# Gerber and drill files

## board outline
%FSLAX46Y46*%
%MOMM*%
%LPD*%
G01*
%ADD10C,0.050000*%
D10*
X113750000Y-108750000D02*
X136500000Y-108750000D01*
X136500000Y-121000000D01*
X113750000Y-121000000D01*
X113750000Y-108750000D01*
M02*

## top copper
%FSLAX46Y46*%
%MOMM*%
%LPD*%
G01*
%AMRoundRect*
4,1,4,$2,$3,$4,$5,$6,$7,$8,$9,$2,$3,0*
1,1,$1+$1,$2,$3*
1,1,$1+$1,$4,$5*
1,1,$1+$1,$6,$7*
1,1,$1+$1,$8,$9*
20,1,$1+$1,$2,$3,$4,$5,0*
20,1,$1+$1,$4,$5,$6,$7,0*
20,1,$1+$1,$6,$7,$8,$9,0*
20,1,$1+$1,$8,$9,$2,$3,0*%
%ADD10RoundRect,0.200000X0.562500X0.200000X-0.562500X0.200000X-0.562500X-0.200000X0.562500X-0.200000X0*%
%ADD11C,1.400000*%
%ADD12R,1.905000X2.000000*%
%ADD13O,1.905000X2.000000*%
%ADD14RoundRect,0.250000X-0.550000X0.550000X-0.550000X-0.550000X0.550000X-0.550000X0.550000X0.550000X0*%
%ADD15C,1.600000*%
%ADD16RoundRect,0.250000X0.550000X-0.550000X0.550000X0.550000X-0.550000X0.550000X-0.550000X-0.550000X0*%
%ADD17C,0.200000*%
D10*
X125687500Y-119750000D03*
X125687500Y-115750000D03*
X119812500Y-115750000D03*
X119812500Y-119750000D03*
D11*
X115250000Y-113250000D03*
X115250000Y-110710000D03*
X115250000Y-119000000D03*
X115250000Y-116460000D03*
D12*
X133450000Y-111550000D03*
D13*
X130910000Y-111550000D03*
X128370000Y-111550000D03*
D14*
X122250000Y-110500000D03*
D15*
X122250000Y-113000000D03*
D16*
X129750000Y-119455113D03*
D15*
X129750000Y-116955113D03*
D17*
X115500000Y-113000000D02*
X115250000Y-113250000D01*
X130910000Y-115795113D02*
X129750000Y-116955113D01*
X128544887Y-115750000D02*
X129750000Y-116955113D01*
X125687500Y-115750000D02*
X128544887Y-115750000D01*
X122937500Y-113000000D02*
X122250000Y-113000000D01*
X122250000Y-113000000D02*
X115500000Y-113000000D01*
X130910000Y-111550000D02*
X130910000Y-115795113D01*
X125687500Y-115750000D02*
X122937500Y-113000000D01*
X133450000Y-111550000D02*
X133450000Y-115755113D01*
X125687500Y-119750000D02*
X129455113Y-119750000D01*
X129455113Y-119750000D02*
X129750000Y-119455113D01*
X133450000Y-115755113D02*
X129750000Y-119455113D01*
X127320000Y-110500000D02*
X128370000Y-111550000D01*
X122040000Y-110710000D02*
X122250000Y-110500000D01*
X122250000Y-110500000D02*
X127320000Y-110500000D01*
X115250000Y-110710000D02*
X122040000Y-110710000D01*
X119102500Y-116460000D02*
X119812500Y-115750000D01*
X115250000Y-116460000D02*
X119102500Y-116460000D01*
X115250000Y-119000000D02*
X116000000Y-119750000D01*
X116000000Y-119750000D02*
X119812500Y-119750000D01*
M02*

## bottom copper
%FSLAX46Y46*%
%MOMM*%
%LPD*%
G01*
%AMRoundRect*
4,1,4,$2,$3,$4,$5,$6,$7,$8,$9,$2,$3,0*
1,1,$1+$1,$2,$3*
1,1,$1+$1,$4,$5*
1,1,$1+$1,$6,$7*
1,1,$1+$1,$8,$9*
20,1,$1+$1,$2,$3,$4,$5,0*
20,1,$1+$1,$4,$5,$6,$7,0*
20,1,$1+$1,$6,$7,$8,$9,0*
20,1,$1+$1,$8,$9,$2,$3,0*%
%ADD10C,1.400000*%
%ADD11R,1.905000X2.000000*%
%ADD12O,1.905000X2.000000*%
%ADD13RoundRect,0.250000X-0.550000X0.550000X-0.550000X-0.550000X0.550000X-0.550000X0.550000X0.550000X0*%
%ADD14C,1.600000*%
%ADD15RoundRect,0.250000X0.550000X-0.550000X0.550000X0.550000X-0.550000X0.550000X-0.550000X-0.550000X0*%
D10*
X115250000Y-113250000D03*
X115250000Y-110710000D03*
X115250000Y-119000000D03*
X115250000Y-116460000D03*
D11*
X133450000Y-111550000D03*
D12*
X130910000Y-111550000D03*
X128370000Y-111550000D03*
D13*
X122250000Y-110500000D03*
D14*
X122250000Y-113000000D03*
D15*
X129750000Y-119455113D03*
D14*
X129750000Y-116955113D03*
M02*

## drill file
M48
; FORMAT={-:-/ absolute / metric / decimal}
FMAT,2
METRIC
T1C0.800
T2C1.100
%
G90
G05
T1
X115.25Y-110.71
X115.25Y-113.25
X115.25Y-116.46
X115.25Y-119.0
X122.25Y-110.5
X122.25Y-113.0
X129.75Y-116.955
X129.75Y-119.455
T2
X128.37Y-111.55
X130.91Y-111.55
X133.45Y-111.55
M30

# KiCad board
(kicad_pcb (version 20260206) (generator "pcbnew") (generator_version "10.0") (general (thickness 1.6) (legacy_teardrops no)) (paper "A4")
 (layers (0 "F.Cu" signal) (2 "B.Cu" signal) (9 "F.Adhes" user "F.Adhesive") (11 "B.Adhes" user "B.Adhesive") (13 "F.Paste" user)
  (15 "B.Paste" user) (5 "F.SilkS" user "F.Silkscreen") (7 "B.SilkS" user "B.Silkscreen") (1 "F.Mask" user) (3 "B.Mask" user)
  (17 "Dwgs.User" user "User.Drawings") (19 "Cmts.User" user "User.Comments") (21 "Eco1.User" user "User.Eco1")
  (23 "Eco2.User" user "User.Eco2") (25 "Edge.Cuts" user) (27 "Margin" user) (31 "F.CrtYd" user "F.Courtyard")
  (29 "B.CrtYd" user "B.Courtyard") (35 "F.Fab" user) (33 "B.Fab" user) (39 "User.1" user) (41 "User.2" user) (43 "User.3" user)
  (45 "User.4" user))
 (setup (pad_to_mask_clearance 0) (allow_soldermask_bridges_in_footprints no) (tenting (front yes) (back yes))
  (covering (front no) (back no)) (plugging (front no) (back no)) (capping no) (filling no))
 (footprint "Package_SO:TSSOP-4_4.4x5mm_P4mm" (layer "F.Cu") (at 122.75 117.75 180)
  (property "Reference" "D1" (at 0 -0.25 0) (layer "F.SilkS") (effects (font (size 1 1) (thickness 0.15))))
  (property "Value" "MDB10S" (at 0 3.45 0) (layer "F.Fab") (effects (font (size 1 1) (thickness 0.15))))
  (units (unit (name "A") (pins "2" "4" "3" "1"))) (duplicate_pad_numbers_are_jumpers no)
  (pad "1" smd roundrect (at -2.9375 -2 180) (size 1.525 0.8) (layers "F.Cu" "F.Mask" "F.Paste") (roundrect_rratio 0.25) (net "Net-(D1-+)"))
  (pad "2" smd roundrect (at -2.9375 2 180) (size 1.525 0.8) (layers "F.Cu" "F.Mask" "F.Paste") (roundrect_rratio 0.25) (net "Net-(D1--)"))
  (pad "3" smd roundrect (at 2.9375 2 180) (size 1.525 0.8) (layers "F.Cu" "F.Mask" "F.Paste") (roundrect_rratio 0.25) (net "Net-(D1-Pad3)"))
  (pad "4" smd roundrect (at 2.9375 -2 180) (size 1.525 0.8) (layers "F.Cu" "F.Mask" "F.Paste") (roundrect_rratio 0.25)
   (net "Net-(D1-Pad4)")))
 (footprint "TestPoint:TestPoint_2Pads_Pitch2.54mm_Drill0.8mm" (layer "F.Cu") (at 115.25 113.25 90)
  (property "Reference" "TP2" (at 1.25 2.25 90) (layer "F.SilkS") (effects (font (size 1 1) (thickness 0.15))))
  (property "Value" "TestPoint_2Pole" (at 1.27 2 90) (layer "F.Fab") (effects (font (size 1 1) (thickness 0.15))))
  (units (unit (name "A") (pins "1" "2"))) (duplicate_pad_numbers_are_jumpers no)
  (pad "1" thru_hole circle (at 0 0 90) (size 1.4 1.4) (drill 0.8) (layers "*.Cu" "*.Mask") (remove_unused_layers no) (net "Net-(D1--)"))
  (pad "2" thru_hole circle (at 2.54 0 90) (size 1.4 1.4) (drill 0.8) (layers "*.Cu" "*.Mask") (remove_unused_layers no)
   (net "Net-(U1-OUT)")))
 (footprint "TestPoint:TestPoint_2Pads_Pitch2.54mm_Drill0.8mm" (layer "F.Cu") (at 115.25 119 90)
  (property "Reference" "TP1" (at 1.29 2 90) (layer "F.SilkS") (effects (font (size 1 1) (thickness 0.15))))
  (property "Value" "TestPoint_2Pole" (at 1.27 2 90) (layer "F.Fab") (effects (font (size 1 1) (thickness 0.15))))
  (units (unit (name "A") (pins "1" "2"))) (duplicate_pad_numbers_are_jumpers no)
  (pad "1" thru_hole circle (at 0 0 90) (size 1.4 1.4) (drill 0.8) (layers "*.Cu" "*.Mask") (remove_unused_layers no) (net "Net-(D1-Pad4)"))
  (pad "2" thru_hole circle (at 2.54 0 90) (size 1.4 1.4) (drill 0.8) (layers "*.Cu" "*.Mask") (remove_unused_layers no)
   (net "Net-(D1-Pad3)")))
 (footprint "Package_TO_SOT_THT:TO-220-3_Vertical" (layer "F.Cu") (at 133.45 111.55 180)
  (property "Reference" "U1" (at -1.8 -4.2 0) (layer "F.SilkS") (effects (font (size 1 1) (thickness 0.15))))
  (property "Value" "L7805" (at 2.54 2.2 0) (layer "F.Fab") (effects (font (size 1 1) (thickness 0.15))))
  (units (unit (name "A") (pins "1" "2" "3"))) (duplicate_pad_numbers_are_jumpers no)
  (pad "1" thru_hole rect (at 0 0 180) (size 1.905 2) (drill 1.1) (layers "*.Cu" "*.Mask") (remove_unused_layers no) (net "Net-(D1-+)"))
  (pad "2" thru_hole oval (at 2.54 0 180) (size 1.905 2) (drill 1.1) (layers "*.Cu" "*.Mask") (remove_unused_layers no) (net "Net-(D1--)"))
  (pad "3" thru_hole oval (at 5.08 0 180) (size 1.905 2) (drill 1.1) (layers "*.Cu" "*.Mask") (remove_unused_layers no) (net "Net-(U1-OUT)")))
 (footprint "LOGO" (layer "F.Cu") (at 135 119.5)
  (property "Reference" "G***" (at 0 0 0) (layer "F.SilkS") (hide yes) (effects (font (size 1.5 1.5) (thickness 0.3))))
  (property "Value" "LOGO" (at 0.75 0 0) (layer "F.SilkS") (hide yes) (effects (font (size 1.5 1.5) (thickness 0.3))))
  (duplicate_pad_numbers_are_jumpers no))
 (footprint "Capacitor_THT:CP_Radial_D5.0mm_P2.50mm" (layer "F.Cu") (at 122.25 110.5 -90)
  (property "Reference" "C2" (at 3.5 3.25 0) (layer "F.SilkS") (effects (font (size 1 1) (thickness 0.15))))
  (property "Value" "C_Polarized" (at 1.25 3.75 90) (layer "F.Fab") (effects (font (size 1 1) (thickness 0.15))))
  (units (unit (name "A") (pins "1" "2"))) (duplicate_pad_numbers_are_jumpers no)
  (pad "1" thru_hole roundrect (at 0 0 270) (size 1.6 1.6) (drill 0.8) (layers "*.Cu" "*.Mask") (remove_unused_layers no)
   (roundrect_rratio 0.15625) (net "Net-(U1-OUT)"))
  (pad "2" thru_hole circle (at 2.5 0 270) (size 1.6 1.6) (drill 0.8) (layers "*.Cu" "*.Mask") (remove_unused_layers no) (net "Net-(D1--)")))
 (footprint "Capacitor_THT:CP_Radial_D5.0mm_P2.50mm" (layer "F.Cu") (at 129.75 119.455113 90)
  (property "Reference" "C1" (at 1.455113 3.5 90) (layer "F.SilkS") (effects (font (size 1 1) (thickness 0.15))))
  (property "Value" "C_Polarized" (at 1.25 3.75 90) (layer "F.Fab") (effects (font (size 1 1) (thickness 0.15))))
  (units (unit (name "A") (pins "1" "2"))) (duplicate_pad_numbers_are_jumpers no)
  (pad "1" thru_hole roundrect (at 0 0 90) (size 1.6 1.6) (drill 0.8) (layers "*.Cu" "*.Mask") (remove_unused_layers no)
   (roundrect_rratio 0.15625) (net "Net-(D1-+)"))
  (pad "2" thru_hole circle (at 2.5 0 90) (size 1.6 1.6) (drill 0.8) (layers "*.Cu" "*.Mask") (remove_unused_layers no) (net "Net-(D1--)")))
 (gr_rect (start 113.75 108.75) (end 136.5 121) (stroke (width 0.05) (type default)) (fill no) (layer "Edge.Cuts"))
 (segment (start 115.5 113) (end 115.25 113.25) (width 0.2) (layer "F.Cu") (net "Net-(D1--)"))
 (segment (start 130.91 115.795113) (end 129.75 116.955113) (width 0.2) (layer "F.Cu") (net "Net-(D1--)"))
 (segment (start 128.544887 115.75) (end 129.75 116.955113) (width 0.2) (layer "F.Cu") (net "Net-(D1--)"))
 (segment (start 125.6875 115.75) (end 128.544887 115.75) (width 0.2) (layer "F.Cu") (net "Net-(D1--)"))
 (segment (start 122.9375 113) (end 122.25 113) (width 0.2) (layer "F.Cu") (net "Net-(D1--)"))
 (segment (start 122.25 113) (end 115.5 113) (width 0.2) (layer "F.Cu") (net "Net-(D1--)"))
 (segment (start 130.91 111.55) (end 130.91 115.795113) (width 0.2) (layer "F.Cu") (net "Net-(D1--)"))
 (segment (start 125.6875 115.75) (end 122.9375 113) (width 0.2) (layer "F.Cu") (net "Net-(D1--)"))
 (segment (start 133.45 111.55) (end 133.45 115.755113) (width 0.2) (layer "F.Cu") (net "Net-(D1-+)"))
 (segment (start 125.6875 119.75) (end 129.455113 119.75) (width 0.2) (layer "F.Cu") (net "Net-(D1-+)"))
 (segment (start 129.455113 119.75) (end 129.75 119.455113) (width 0.2) (layer "F.Cu") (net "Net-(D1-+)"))
 (segment (start 133.45 115.755113) (end 129.75 119.455113) (width 0.2) (layer "F.Cu") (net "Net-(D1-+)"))
 (segment (start 127.32 110.5) (end 128.37 111.55) (width 0.2) (layer "F.Cu") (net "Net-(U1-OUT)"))
 (segment (start 122.04 110.71) (end 122.25 110.5) (width 0.2) (layer "F.Cu") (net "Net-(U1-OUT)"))
 (segment (start 122.25 110.5) (end 127.32 110.5) (width 0.2) (layer "F.Cu") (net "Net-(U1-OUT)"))
 (segment (start 115.25 110.71) (end 122.04 110.71) (width 0.2) (layer "F.Cu") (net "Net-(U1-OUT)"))
 (segment (start 119.1025 116.46) (end 119.8125 115.75) (width 0.2) (layer "F.Cu") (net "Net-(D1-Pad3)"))
 (segment (start 115.25 116.46) (end 119.1025 116.46) (width 0.2) (layer "F.Cu") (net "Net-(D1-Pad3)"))
 (segment (start 115.25 119) (end 116 119.75) (width 0.2) (layer "F.Cu") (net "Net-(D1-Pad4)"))
 (segment (start 116 119.75) (end 119.8125 119.75) (width 0.2) (layer "F.Cu") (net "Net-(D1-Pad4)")))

